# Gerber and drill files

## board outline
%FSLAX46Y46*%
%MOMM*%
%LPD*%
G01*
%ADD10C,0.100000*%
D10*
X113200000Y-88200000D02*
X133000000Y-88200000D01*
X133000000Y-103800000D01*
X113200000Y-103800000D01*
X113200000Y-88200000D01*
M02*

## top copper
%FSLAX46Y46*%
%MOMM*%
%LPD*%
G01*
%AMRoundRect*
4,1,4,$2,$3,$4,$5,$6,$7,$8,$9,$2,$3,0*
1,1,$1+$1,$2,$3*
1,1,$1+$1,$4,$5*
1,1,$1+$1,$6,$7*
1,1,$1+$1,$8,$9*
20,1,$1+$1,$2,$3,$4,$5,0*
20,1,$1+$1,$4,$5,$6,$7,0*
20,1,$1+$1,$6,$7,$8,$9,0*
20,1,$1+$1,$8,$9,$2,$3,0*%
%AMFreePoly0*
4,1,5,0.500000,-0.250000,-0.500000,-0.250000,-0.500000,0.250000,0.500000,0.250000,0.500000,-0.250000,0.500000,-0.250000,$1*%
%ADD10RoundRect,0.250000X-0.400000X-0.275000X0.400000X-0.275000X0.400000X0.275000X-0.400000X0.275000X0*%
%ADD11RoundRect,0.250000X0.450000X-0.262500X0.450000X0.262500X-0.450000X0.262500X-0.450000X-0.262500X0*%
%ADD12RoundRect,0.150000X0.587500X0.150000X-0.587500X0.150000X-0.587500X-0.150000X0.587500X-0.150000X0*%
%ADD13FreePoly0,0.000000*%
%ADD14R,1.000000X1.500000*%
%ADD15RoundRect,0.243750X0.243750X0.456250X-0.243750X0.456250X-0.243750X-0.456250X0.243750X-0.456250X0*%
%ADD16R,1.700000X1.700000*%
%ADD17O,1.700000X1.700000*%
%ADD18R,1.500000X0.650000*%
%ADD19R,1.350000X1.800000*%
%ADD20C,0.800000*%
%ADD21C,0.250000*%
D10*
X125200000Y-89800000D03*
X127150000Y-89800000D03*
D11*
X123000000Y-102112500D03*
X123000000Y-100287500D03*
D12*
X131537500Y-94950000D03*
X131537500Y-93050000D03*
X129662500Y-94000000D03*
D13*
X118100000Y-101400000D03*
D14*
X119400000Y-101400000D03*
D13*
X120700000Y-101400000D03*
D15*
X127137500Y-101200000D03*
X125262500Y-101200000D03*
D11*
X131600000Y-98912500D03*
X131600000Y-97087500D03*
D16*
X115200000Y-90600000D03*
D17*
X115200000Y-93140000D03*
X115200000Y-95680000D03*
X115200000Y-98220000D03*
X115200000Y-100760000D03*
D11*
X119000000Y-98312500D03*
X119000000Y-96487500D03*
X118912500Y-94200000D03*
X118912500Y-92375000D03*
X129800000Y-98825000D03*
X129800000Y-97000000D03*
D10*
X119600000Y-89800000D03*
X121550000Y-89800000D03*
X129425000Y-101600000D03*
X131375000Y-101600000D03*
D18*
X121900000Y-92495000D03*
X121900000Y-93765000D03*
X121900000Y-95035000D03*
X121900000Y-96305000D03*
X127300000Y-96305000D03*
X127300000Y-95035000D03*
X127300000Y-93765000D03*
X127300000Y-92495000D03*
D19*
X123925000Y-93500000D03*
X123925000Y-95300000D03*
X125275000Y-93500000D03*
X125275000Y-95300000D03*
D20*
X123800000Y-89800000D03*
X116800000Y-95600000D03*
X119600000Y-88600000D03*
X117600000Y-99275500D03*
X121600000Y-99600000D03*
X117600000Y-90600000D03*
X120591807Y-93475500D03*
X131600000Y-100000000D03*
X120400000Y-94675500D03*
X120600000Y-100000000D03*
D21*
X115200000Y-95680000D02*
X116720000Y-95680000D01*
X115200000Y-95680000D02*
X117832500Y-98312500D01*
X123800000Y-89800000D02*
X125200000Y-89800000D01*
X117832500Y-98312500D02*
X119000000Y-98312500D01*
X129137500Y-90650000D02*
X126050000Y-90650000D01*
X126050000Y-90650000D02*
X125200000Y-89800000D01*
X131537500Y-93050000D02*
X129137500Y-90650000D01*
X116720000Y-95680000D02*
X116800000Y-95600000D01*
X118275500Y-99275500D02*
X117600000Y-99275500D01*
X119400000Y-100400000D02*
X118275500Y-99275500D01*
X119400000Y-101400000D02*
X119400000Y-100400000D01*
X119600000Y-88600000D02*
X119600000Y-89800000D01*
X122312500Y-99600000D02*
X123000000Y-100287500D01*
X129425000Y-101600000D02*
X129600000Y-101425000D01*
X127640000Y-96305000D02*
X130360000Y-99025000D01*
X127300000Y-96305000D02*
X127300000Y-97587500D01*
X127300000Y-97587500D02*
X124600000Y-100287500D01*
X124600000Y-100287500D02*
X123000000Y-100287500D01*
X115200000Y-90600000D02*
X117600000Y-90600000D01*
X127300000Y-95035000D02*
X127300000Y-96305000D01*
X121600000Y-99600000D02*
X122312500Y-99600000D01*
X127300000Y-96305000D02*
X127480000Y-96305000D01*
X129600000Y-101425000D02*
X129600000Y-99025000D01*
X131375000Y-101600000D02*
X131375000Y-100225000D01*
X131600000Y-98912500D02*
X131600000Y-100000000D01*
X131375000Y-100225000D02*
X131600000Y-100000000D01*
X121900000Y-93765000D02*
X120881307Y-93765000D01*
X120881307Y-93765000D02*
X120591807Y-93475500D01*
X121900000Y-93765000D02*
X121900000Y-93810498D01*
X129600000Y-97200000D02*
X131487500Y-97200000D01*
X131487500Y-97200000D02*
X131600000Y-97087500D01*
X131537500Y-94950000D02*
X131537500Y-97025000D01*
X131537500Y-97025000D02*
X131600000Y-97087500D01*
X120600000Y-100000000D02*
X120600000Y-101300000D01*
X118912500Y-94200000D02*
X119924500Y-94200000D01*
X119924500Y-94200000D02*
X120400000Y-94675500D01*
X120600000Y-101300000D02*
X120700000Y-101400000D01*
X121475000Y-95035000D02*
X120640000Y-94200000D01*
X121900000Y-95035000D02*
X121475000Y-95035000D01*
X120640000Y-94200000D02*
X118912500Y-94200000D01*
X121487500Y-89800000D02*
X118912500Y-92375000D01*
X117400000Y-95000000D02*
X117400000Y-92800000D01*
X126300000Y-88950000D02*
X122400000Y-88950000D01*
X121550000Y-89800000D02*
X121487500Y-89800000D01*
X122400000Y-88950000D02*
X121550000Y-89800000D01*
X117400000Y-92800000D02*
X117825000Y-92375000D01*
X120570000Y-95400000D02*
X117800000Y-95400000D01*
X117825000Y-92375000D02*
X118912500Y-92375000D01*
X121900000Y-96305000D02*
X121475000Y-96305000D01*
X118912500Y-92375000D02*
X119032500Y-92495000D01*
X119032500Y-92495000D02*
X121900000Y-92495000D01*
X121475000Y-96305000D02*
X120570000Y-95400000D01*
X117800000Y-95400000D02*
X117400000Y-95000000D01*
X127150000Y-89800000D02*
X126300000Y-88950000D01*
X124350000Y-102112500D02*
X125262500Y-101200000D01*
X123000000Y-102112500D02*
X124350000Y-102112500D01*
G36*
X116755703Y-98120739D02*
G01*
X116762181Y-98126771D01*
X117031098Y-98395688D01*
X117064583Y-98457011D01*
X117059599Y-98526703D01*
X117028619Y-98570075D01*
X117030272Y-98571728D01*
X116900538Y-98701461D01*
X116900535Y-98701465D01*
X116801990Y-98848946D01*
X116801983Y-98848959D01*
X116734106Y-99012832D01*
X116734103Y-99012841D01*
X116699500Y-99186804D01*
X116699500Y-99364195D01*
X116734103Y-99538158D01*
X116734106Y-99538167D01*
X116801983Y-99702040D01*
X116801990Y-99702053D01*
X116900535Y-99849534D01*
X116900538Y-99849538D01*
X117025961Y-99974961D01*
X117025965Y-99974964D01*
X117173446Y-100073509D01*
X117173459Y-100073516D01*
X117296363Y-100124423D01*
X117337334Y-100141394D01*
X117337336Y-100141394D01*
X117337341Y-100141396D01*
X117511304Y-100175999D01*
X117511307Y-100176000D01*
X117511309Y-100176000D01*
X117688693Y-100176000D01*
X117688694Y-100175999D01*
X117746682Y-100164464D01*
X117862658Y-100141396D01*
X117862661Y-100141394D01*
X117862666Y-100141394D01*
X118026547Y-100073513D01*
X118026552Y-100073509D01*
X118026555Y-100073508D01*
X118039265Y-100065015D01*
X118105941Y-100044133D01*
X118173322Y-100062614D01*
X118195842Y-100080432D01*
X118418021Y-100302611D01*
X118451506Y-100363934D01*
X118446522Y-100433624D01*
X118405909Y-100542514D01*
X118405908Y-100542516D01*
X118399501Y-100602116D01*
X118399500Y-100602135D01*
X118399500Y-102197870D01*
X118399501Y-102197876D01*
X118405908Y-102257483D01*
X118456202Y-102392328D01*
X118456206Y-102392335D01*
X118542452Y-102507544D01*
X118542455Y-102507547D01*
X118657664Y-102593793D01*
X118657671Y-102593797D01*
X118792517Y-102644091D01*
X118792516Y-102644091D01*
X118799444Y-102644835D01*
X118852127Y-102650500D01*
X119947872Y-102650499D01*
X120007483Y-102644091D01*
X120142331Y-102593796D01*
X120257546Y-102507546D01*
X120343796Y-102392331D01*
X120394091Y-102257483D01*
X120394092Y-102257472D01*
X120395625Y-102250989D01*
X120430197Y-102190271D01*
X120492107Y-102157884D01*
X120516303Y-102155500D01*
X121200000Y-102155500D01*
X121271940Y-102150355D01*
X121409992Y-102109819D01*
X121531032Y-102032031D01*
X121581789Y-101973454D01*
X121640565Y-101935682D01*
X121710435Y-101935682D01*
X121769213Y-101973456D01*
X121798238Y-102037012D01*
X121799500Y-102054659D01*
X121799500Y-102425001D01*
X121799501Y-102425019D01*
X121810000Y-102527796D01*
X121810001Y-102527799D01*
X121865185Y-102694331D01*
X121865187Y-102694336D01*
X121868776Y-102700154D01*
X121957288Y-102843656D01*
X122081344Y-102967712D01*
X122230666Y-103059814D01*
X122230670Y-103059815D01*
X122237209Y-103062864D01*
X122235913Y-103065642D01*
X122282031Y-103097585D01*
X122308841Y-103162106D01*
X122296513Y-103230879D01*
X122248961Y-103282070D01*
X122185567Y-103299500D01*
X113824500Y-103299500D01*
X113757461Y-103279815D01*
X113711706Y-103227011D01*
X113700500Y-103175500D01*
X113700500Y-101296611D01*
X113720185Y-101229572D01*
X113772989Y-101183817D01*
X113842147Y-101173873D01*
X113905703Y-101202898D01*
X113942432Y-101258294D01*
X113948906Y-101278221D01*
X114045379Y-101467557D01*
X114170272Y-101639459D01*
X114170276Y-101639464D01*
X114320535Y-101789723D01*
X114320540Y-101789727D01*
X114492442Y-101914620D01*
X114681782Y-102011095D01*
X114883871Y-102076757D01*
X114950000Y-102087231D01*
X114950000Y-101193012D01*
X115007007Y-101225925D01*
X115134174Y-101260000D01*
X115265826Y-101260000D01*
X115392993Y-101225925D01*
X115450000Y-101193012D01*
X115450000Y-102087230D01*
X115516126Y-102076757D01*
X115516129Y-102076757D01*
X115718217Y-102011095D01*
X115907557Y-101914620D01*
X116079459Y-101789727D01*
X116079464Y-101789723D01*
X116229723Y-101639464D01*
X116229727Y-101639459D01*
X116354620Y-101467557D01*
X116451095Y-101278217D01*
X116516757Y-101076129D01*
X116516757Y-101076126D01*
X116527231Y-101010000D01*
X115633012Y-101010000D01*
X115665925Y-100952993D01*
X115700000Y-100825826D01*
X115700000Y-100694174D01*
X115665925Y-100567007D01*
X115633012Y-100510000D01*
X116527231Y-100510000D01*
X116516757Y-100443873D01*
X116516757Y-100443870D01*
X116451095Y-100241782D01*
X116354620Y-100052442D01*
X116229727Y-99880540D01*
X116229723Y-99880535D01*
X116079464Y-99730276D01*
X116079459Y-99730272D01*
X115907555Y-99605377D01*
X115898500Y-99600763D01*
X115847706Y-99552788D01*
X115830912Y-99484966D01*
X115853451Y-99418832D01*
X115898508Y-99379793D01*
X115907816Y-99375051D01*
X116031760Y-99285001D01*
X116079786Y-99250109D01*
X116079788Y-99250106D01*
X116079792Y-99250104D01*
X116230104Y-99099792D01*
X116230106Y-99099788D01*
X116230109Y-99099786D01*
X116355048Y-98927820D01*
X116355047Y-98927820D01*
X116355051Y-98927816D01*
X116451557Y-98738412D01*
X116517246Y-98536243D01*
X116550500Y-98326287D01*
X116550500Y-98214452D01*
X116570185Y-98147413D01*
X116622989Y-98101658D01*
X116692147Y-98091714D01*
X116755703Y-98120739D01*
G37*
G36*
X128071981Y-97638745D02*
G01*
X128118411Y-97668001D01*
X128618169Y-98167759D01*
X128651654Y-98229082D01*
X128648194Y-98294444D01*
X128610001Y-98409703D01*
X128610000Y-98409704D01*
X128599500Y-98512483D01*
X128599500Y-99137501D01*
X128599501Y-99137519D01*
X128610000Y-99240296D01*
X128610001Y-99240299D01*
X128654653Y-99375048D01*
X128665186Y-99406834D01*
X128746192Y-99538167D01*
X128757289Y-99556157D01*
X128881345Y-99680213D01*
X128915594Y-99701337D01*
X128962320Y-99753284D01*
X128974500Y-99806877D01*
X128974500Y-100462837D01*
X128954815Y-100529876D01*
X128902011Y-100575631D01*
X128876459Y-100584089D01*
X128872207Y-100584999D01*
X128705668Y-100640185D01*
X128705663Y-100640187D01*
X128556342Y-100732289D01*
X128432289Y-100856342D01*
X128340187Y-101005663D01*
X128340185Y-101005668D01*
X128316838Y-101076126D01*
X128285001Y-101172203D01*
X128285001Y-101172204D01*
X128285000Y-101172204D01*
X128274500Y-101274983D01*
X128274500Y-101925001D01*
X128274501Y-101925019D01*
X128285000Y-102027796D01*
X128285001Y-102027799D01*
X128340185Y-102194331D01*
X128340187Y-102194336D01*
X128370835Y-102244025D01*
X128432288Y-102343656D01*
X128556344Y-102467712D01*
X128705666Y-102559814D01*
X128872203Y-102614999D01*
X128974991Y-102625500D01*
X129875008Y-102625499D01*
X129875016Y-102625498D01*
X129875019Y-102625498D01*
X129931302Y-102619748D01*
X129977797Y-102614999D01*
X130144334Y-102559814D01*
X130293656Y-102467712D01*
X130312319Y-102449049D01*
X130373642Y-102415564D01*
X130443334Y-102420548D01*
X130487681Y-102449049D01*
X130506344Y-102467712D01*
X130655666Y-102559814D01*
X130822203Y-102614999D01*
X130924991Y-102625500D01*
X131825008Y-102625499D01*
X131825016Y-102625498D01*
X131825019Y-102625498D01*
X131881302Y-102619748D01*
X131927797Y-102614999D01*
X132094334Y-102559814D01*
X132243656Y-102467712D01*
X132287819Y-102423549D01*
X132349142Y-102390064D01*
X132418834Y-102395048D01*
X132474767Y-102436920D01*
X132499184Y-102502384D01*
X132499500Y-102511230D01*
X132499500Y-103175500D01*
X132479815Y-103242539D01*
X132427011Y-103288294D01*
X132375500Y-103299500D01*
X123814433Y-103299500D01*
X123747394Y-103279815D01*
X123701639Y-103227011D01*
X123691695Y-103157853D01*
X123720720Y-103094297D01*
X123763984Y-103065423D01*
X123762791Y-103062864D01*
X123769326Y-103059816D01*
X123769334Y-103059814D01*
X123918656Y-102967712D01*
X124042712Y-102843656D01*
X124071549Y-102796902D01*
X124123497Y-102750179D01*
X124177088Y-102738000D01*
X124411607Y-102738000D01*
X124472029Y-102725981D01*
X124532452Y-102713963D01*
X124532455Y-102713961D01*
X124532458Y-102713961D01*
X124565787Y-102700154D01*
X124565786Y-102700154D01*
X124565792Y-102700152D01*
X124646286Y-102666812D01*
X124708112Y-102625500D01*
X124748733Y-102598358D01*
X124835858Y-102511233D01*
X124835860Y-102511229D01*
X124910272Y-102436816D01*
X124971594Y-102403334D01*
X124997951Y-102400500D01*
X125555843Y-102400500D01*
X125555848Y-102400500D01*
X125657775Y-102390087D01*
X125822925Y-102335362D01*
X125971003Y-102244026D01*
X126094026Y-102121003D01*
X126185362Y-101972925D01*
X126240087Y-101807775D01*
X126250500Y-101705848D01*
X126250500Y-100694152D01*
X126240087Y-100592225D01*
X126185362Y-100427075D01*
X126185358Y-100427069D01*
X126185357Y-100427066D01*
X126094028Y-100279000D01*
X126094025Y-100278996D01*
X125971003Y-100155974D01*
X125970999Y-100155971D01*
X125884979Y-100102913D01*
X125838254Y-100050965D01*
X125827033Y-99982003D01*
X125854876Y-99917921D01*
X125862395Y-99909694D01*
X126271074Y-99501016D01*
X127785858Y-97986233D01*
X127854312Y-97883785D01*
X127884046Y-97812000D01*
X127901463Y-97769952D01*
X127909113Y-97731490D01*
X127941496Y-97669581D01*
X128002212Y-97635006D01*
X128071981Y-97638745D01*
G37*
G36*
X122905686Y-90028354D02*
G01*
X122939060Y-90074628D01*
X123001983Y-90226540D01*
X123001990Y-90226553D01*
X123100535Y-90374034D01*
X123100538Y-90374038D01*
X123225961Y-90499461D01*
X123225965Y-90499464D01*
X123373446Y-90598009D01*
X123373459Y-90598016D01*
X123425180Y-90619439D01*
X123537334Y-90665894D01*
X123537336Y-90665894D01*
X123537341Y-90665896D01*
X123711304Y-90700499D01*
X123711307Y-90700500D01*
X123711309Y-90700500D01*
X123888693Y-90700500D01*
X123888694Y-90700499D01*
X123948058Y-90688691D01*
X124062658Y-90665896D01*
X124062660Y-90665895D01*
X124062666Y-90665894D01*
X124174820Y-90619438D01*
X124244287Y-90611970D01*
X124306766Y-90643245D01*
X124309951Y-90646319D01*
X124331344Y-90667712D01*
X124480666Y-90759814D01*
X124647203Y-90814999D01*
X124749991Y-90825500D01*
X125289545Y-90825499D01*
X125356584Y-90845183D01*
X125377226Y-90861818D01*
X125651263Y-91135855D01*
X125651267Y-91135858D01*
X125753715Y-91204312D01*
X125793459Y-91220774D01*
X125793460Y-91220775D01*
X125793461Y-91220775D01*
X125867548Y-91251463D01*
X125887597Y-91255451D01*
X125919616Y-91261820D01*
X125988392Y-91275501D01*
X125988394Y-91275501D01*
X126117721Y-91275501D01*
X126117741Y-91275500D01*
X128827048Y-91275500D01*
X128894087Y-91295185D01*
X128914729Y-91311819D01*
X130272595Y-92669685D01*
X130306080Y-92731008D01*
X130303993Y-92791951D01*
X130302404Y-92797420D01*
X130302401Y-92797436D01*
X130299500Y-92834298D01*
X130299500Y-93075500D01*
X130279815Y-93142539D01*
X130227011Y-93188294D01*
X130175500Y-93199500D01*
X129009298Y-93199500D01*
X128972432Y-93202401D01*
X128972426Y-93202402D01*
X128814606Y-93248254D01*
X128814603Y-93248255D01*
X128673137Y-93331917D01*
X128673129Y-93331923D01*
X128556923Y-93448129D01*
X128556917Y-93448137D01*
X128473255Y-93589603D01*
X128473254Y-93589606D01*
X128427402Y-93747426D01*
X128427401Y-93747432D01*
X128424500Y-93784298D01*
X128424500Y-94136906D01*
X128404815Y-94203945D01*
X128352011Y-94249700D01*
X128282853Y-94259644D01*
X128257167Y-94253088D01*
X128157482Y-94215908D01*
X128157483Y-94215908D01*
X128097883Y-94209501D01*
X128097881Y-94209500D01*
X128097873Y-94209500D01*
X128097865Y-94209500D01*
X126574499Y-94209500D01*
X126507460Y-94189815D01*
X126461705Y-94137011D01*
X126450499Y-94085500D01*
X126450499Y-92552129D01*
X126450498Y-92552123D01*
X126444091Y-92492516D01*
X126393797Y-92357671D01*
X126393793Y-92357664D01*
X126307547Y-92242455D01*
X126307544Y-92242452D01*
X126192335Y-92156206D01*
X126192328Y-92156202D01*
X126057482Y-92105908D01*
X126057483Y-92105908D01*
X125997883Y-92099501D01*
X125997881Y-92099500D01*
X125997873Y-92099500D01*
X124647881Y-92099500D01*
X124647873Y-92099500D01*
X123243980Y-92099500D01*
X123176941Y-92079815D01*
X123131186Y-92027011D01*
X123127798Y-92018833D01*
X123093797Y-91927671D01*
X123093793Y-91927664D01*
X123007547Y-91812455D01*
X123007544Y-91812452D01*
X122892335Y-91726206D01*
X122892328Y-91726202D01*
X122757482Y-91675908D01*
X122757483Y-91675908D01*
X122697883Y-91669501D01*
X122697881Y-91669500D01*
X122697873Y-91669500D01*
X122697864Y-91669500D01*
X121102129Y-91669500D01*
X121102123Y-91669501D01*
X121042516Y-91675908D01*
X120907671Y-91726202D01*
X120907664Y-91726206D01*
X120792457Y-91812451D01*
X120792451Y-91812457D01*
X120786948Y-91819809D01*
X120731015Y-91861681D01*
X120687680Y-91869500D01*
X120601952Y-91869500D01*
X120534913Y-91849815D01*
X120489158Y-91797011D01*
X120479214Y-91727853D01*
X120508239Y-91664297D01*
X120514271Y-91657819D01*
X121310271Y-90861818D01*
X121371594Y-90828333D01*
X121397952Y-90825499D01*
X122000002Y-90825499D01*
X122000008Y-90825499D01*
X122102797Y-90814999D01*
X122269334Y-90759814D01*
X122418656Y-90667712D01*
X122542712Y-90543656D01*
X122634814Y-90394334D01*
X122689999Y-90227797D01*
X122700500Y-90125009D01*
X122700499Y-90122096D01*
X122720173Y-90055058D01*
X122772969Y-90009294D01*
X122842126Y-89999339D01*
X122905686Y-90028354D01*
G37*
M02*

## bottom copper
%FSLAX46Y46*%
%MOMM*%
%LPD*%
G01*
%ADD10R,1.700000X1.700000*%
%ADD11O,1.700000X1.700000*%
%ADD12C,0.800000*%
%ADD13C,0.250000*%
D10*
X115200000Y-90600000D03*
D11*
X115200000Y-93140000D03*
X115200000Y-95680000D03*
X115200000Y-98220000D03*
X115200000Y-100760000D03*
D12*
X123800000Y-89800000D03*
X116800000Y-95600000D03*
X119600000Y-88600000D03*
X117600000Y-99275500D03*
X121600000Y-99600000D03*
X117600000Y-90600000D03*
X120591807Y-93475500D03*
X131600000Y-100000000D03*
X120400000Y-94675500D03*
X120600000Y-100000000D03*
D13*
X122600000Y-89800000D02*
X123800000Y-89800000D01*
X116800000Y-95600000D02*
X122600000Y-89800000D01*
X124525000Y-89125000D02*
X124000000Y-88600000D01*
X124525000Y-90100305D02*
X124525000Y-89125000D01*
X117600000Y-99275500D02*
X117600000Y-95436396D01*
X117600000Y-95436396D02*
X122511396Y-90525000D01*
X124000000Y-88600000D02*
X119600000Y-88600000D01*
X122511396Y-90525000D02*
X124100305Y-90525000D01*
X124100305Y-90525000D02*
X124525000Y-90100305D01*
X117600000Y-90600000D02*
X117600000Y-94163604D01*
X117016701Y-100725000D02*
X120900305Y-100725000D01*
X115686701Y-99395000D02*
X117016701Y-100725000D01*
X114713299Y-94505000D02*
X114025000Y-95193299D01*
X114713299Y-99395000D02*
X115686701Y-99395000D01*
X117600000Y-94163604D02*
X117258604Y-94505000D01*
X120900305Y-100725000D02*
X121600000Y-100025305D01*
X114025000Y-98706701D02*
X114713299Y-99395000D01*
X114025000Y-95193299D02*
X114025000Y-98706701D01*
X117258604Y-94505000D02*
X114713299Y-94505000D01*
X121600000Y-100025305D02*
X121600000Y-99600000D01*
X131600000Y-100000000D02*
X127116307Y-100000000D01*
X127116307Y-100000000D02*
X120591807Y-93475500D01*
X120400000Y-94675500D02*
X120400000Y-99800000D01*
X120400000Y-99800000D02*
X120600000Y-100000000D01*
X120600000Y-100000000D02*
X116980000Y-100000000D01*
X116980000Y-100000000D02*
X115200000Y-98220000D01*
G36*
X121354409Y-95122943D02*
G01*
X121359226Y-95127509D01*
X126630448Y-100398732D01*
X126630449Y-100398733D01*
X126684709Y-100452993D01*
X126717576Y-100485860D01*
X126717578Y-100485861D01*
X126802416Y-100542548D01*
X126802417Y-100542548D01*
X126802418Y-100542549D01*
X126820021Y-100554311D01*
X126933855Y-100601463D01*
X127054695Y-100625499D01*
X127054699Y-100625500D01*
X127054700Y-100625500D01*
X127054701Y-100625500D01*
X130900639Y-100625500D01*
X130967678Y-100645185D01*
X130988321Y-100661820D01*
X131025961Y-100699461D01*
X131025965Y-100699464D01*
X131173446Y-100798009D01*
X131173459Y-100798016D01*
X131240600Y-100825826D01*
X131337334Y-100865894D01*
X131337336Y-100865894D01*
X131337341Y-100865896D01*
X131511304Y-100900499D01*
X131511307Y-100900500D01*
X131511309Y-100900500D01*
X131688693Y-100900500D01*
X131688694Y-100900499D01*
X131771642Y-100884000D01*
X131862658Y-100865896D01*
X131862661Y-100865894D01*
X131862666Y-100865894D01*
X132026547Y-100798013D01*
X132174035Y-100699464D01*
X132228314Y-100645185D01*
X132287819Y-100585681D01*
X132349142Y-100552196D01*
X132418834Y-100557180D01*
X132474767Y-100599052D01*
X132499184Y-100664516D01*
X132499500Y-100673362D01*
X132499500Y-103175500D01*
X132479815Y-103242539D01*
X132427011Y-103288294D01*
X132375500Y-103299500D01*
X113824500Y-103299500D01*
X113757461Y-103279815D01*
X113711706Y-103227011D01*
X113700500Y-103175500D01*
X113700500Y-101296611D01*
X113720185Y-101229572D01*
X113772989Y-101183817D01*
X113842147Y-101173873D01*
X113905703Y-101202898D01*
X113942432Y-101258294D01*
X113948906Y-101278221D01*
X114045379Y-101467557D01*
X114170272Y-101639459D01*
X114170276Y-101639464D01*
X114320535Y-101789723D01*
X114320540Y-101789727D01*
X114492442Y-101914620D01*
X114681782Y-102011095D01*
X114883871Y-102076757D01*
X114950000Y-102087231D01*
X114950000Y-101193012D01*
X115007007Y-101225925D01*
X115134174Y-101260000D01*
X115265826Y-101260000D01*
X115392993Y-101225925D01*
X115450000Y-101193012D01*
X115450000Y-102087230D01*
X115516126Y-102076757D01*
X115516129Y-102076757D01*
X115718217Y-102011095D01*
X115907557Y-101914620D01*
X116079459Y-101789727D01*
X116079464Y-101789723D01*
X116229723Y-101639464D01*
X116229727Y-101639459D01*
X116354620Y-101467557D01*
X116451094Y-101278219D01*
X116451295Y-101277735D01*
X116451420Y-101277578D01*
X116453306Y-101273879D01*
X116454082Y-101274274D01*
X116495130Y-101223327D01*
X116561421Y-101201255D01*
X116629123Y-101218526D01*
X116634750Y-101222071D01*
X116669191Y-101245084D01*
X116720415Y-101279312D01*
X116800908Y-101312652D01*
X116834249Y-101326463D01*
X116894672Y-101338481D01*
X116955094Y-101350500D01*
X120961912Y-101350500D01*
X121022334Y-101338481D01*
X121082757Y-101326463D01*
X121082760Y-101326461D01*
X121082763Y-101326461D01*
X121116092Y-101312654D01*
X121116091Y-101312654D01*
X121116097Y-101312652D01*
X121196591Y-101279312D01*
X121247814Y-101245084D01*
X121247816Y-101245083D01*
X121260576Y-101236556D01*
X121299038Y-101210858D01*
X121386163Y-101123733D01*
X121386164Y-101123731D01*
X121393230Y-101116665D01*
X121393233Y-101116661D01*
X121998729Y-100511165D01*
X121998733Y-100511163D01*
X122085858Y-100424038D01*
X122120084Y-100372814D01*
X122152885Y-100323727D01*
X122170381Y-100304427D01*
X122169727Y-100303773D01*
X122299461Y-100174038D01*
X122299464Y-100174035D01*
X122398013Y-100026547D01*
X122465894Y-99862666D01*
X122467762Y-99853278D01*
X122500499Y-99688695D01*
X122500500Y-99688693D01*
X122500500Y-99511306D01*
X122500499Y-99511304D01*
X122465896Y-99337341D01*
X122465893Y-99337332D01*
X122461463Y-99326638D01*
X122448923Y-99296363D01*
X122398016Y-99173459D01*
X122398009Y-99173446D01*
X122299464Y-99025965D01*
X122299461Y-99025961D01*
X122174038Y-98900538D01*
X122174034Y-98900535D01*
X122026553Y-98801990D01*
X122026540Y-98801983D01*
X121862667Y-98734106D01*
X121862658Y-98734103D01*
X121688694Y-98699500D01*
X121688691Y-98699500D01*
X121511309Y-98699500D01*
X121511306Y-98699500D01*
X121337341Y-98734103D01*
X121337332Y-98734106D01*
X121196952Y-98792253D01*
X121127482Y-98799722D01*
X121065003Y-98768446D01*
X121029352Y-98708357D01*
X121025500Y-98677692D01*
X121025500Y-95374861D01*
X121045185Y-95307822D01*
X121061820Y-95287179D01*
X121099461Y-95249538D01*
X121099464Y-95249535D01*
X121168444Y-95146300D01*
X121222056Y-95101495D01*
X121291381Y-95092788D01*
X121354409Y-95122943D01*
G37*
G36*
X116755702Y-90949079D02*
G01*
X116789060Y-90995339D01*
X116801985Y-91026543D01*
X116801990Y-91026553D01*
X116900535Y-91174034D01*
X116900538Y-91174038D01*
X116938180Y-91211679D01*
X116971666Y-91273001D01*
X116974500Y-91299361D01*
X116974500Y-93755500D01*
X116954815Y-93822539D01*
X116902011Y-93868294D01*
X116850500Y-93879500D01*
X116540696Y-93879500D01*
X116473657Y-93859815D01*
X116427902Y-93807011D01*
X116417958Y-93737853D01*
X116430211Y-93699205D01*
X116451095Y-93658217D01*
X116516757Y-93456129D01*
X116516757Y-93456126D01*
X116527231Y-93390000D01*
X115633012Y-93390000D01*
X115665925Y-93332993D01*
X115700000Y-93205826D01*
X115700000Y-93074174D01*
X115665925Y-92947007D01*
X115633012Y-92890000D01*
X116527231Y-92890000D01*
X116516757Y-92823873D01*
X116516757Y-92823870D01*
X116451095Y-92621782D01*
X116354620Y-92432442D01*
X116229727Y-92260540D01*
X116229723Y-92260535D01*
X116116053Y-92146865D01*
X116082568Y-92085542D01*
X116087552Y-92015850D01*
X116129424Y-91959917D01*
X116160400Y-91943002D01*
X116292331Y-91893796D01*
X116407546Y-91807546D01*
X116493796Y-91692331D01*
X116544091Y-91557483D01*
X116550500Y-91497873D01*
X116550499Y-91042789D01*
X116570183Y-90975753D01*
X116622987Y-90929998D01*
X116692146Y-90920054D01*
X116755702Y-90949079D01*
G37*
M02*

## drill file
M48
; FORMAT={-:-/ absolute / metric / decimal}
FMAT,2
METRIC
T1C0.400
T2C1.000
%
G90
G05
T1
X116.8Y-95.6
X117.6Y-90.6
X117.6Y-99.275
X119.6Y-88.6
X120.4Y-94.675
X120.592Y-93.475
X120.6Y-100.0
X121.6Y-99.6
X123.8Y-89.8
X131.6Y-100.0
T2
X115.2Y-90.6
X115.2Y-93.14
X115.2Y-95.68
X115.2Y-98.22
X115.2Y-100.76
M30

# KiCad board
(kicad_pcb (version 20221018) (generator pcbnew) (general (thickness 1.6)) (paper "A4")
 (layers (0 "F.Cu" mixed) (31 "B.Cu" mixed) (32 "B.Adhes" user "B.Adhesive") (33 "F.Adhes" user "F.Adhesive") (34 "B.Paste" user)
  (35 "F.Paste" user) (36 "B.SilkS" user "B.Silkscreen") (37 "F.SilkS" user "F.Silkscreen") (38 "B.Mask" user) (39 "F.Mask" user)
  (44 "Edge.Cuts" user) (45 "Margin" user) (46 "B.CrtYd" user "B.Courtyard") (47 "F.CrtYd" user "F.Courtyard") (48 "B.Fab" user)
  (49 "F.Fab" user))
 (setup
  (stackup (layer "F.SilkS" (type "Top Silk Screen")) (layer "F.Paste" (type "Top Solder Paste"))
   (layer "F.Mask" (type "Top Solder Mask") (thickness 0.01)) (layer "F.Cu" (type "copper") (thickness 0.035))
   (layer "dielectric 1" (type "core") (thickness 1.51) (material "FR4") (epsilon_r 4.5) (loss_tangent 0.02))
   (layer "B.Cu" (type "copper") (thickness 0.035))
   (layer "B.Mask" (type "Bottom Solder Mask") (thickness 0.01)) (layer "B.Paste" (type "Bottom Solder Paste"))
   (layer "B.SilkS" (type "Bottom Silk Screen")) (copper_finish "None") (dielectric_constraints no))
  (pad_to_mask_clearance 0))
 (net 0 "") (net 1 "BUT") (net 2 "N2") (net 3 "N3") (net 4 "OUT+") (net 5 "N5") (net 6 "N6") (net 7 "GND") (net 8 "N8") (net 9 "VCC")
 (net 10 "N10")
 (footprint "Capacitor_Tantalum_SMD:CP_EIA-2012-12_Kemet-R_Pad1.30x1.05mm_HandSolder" (layer "F.Cu") (at 126.175 89.8)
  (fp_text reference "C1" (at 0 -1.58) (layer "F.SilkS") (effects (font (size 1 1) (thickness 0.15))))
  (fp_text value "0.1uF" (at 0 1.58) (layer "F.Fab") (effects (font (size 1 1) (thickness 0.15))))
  (pad "1" smd roundrect (at -0.975 0) (size 1.3 1.05) (layers "F.Cu" "F.Paste" "F.Mask") (roundrect_rratio 0.2380952381) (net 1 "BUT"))
  (pad "2" smd roundrect (at 0.975 0) (size 1.3 1.05) (layers "F.Cu" "F.Paste" "F.Mask") (roundrect_rratio 0.2380952381) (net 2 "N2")))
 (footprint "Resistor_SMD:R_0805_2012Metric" (layer "F.Cu") (at 123 101.2 90)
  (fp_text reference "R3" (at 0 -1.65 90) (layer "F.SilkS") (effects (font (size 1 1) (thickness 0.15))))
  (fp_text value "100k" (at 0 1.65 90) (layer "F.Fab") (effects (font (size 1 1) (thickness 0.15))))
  (pad "1" smd roundrect (at -0.9125 0 90) (size 1.025 1.4) (layers "F.Cu" "F.Paste" "F.Mask") (roundrect_rratio 0.243902439) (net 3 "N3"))
  (pad "2" smd roundrect (at 0.9125 0 90) (size 1.025 1.4) (layers "F.Cu" "F.Paste" "F.Mask") (roundrect_rratio 0.243902439) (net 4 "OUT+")))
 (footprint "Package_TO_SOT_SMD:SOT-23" (layer "F.Cu") (at 130.6 94 180)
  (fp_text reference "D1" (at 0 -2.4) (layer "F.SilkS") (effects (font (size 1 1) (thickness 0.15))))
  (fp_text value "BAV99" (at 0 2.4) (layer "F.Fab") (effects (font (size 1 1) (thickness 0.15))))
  (pad "1" smd roundrect (at -0.9375 -0.95 180) (size 1.475 0.6) (layers "F.Cu" "F.Paste" "F.Mask") (roundrect_rratio 0.25) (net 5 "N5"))
  (pad "2" smd roundrect (at -0.9375 0.95 180) (size 1.475 0.6) (layers "F.Cu" "F.Paste" "F.Mask") (roundrect_rratio 0.25) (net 1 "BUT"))
  (pad "3" smd roundrect (at 0.9375 0 180) (size 1.475 0.6) (layers "F.Cu" "F.Paste" "F.Mask") (roundrect_rratio 0.25) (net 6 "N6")))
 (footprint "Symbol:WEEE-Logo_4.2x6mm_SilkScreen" (layer "F.Cu") (at 126 98.4)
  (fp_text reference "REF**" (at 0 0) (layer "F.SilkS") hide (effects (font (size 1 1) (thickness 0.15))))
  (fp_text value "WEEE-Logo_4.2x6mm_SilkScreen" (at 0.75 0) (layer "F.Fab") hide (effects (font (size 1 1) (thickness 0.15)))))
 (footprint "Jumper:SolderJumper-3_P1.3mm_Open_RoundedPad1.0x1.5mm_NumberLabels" (layer "F.Cu") (at 119.4 101.4)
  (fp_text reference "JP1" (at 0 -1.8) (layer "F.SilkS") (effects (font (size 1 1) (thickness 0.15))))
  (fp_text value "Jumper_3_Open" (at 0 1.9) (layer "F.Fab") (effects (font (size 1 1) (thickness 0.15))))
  (pad "1" smd custom (at -1.3 0) (size 1 0.5) (layers "F.Cu" "F.Mask") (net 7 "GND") (zone_connect 2) (thermal_bridge_angle 45)
   (options (clearance outline) (anchor rect)) (primitives))
  (pad "2" smd rect (at 0 0) (size 1 1.5) (layers "F.Cu" "F.Mask") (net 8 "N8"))
  (pad "3" smd custom (at 1.3 0) (size 1 0.5) (layers "F.Cu" "F.Mask") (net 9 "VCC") (zone_connect 2) (thermal_bridge_angle 45)
   (options (clearance outline) (anchor rect)) (primitives)))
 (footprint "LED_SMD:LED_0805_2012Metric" (layer "F.Cu") (at 126.2 101.2 180)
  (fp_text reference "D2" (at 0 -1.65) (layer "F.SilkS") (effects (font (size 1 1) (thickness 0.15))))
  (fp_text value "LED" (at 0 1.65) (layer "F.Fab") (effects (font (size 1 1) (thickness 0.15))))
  (pad "1" smd roundrect (at -0.9375 0 180) (size 0.975 1.4) (layers "F.Cu" "F.Paste" "F.Mask") (roundrect_rratio 0.25) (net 7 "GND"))
  (pad "2" smd roundrect (at 0.9375 0 180) (size 0.975 1.4) (layers "F.Cu" "F.Paste" "F.Mask") (roundrect_rratio 0.25) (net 3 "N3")))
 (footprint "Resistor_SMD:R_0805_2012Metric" (layer "F.Cu") (at 131.6 98 90)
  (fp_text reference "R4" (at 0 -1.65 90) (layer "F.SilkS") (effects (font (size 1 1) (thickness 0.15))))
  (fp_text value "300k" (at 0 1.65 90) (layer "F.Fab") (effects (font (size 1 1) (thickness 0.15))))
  (pad "1" smd roundrect (at -0.9125 0 90) (size 1.025 1.4) (layers "F.Cu" "F.Paste" "F.Mask") (roundrect_rratio 0.243902439) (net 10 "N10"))
  (pad "2" smd roundrect (at 0.9125 0 90) (size 1.025 1.4) (layers "F.Cu" "F.Paste" "F.Mask") (roundrect_rratio 0.243902439) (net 5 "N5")))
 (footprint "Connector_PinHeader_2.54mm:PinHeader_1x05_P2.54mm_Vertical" (layer "F.Cu") (at 115.2 90.6)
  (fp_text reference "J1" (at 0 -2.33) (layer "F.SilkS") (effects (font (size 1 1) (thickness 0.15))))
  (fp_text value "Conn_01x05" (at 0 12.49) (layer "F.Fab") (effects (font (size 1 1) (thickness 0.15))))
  (pad "1" thru_hole rect (at 0 0) (size 1.7 1.7) (drill 1) (layers "*.Cu" "*.Mask") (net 4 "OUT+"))
  (pad "2" thru_hole oval (at 0 2.54) (size 1.7 1.7) (drill 1) (layers "*.Cu" "*.Mask") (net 7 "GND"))
  (pad "3" thru_hole oval (at 0 5.08) (size 1.7 1.7) (drill 1) (layers "*.Cu" "*.Mask") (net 1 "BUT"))
  (pad "4" thru_hole oval (at 0 7.62) (size 1.7 1.7) (drill 1) (layers "*.Cu" "*.Mask") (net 9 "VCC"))
  (pad "5" thru_hole oval (at 0 10.16) (size 1.7 1.7) (drill 1) (layers "*.Cu" "*.Mask") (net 7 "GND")))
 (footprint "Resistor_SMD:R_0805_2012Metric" (layer "F.Cu") (at 119 97.4 90)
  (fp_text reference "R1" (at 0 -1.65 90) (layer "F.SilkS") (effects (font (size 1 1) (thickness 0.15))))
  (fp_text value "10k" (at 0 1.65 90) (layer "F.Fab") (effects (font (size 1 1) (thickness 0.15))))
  (pad "1" smd roundrect (at -0.9125 0 90) (size 1.025 1.4) (layers "F.Cu" "F.Paste" "F.Mask") (roundrect_rratio 0.243902439) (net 1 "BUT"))
  (pad "2" smd roundrect (at 0.9125 0 90) (size 1.025 1.4) (layers "F.Cu" "F.Paste" "F.Mask") (roundrect_rratio 0.243902439) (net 9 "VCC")))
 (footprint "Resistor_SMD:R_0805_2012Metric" (layer "F.Cu") (at 118.9125 93.2875 90)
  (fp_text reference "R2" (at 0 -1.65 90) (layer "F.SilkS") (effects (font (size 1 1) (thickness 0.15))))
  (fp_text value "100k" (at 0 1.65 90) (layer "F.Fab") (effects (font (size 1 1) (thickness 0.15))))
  (pad "1" smd roundrect (at -0.9125 0 90) (size 1.025 1.4) (layers "F.Cu" "F.Paste" "F.Mask") (roundrect_rratio 0.243902439) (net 9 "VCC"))
  (pad "2" smd roundrect (at 0.9125 0 90) (size 1.025 1.4) (layers "F.Cu" "F.Paste" "F.Mask") (roundrect_rratio 0.243902439) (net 2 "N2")))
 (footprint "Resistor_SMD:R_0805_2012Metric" (layer "F.Cu") (at 129.8 97.9125 90)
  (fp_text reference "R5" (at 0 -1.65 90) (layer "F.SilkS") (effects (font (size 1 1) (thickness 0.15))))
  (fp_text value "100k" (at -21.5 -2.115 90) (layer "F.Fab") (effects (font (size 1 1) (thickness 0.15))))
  (pad "1" smd roundrect (at -0.9125 0 90) (size 1.025 1.4) (layers "F.Cu" "F.Paste" "F.Mask") (roundrect_rratio 0.243902439) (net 4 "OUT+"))
  (pad "2" smd roundrect (at 0.9125 0 90) (size 1.025 1.4) (layers "F.Cu" "F.Paste" "F.Mask") (roundrect_rratio 0.243902439) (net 5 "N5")))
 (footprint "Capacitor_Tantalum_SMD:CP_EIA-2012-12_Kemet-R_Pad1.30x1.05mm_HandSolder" (layer "F.Cu") (at 120.575 89.8)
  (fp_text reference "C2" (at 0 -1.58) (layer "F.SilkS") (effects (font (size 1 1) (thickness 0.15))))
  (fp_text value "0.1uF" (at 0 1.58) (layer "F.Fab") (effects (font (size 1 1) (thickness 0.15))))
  (pad "1" smd roundrect (at -0.975 0) (size 1.3 1.05) (layers "F.Cu" "F.Paste" "F.Mask") (roundrect_rratio 0.2380952381) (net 8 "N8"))
  (pad "2" smd roundrect (at 0.975 0) (size 1.3 1.05) (layers "F.Cu" "F.Paste" "F.Mask") (roundrect_rratio 0.2380952381) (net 2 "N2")))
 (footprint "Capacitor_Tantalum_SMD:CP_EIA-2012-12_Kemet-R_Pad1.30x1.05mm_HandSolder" (layer "F.Cu") (at 130.4 101.6)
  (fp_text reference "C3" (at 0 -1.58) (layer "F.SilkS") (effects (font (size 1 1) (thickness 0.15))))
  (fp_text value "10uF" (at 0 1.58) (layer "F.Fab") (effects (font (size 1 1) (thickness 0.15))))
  (pad "1" smd roundrect (at -0.975 0) (size 1.3 1.05) (layers "F.Cu" "F.Paste" "F.Mask") (roundrect_rratio 0.2380952381) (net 4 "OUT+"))
  (pad "2" smd roundrect (at 0.975 0) (size 1.3 1.05) (layers "F.Cu" "F.Paste" "F.Mask") (roundrect_rratio 0.2380952381) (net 10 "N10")))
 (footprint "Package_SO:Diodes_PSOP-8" (layer "F.Cu") (at 124.6 94.4)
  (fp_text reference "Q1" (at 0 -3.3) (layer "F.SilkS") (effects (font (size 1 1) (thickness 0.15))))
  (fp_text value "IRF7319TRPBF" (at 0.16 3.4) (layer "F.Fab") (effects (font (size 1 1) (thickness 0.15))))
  (pad "1" smd rect (at -2.7 -1.905) (size 1.5 0.65) (layers "F.Cu" "F.Paste" "F.Mask") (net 2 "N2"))
  (pad "2" smd rect (at -2.7 -0.635) (size 1.5 0.65) (layers "F.Cu" "F.Paste" "F.Mask") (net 10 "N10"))
  (pad "3" smd rect (at -2.7 0.635) (size 1.5 0.65) (layers "F.Cu" "F.Paste" "F.Mask") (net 9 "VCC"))
  (pad "4" smd rect (at -2.7 1.905) (size 1.5 0.65) (layers "F.Cu" "F.Paste" "F.Mask") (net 2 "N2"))
  (pad "5" smd rect (at 2.7 1.905) (size 1.5 0.65) (layers "F.Cu" "F.Paste" "F.Mask") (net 4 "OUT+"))
  (pad "6" smd rect (at 2.7 0.635) (size 1.5 0.65) (layers "F.Cu" "F.Paste" "F.Mask") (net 4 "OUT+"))
  (pad "7" smd rect (at 2.7 -0.635) (size 1.5 0.65) (layers "F.Cu" "F.Paste" "F.Mask") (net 7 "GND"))
  (pad "8" smd rect (at 2.7 -1.905) (size 1.5 0.65) (layers "F.Cu" "F.Paste" "F.Mask") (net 7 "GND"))
  (pad "9" smd rect (at -0.675 -0.9) (size 1.35 1.8) (layers "F.Cu" "F.Paste" "F.Mask") (solder_paste_margin_ratio -0.2))
  (pad "9" smd rect (at -0.675 0.9) (size 1.35 1.8) (layers "F.Cu" "F.Paste" "F.Mask") (solder_paste_margin_ratio -0.2))
  (pad "9" smd rect (at 0.675 -0.9) (size 1.35 1.8) (layers "F.Cu" "F.Paste" "F.Mask") (solder_paste_margin_ratio -0.2))
  (pad "9" smd rect (at 0.675 0.9) (size 1.35 1.8) (layers "F.Cu" "F.Paste" "F.Mask") (solder_paste_margin_ratio -0.2)))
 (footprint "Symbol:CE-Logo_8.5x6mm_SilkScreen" (layer "B.Cu") (at 127.6 92 180)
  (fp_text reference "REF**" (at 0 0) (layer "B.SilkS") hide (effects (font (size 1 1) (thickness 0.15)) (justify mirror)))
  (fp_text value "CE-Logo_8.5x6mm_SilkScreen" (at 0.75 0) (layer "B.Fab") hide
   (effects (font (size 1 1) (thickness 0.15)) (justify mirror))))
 (gr_rect (start 113.2 88.2) (end 133 103.8) (stroke (width 0.1) (type default)) (fill none) (layer "Edge.Cuts"))
 (segment (start 115.2 95.68) (end 116.72 95.68) (width 0.25) (layer "F.Cu") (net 1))
 (segment (start 115.2 95.68) (end 117.8325 98.3125) (width 0.25) (layer "F.Cu") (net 1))
 (segment (start 123.8 89.8) (end 125.2 89.8) (width 0.25) (layer "F.Cu") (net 1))
 (segment (start 117.8325 98.3125) (end 119 98.3125) (width 0.25) (layer "F.Cu") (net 1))
 (segment (start 129.1375 90.65) (end 126.05 90.65) (width 0.25) (layer "F.Cu") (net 1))
 (segment (start 126.05 90.65) (end 125.2 89.8) (width 0.25) (layer "F.Cu") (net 1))
 (segment (start 131.5375 93.05) (end 129.1375 90.65) (width 0.25) (layer "F.Cu") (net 1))
 (segment (start 116.72 95.68) (end 116.8 95.6) (width 0.25) (layer "F.Cu") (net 1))
 (via (at 123.8 89.8) (size 0.8) (drill 0.4) (layers "F.Cu" "B.Cu") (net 1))
 (via (at 116.8 95.6) (size 0.8) (drill 0.4) (layers "F.Cu" "B.Cu") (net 1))
 (segment (start 122.6 89.8) (end 123.8 89.8) (width 0.25) (layer "B.Cu") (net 1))
 (segment (start 116.8 95.6) (end 122.6 89.8) (width 0.25) (layer "B.Cu") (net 1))
 (segment (start 118.2755 99.2755) (end 117.6 99.2755) (width 0.25) (layer "F.Cu") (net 8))
 (segment (start 119.4 100.4) (end 118.2755 99.2755) (width 0.25) (layer "F.Cu") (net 8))
 (segment (start 119.4 101.4) (end 119.4 100.4) (width 0.25) (layer "F.Cu") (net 8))
 (segment (start 119.6 88.6) (end 119.6 89.8) (width 0.25) (layer "F.Cu") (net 8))
 (via (at 119.6 88.6) (size 0.8) (drill 0.4) (layers "F.Cu" "B.Cu") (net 8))
 (via (at 117.6 99.2755) (size 0.8) (drill 0.4) (layers "F.Cu" "B.Cu") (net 8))
 (segment (start 124.525 89.125) (end 124 88.6) (width 0.25) (layer "B.Cu") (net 8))
 (segment (start 124.525 90.100305) (end 124.525 89.125) (width 0.25) (layer "B.Cu") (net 8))
 (segment (start 117.6 99.2755) (end 117.6 95.436396) (width 0.25) (layer "B.Cu") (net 8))
 (segment (start 117.6 95.436396) (end 122.511396 90.525) (width 0.25) (layer "B.Cu") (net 8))
 (segment (start 124 88.6) (end 119.6 88.6) (width 0.25) (layer "B.Cu") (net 8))
 (segment (start 122.511396 90.525) (end 124.100305 90.525) (width 0.25) (layer "B.Cu") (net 8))
 (segment (start 124.100305 90.525) (end 124.525 90.100305) (width 0.25) (layer "B.Cu") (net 8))
 (segment (start 122.3125 99.6) (end 123 100.2875) (width 0.25) (layer "F.Cu") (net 4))
 (segment (start 129.425 101.6) (end 129.6 101.425) (width 0.25) (layer "F.Cu") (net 4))
 (segment (start 127.64 96.305) (end 130.36 99.025) (width 0.25) (layer "F.Cu") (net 4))
 (segment (start 127.3 96.305) (end 127.3 97.5875) (width 0.25) (layer "F.Cu") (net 4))
 (segment (start 127.3 97.5875) (end 124.6 100.2875) (width 0.25) (layer "F.Cu") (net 4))
 (segment (start 124.6 100.2875) (end 123 100.2875) (width 0.25) (layer "F.Cu") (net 4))
 (segment (start 115.2 90.6) (end 117.6 90.6) (width 0.25) (layer "F.Cu") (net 4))
 (segment (start 127.3 95.035) (end 127.3 96.305) (width 0.25) (layer "F.Cu") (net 4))
 (segment (start 121.6 99.6) (end 122.3125 99.6) (width 0.25) (layer "F.Cu") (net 4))
 (segment (start 127.3 96.305) (end 127.48 96.305) (width 0.25) (layer "F.Cu") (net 4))
 (segment (start 129.6 101.425) (end 129.6 99.025) (width 0.25) (layer "F.Cu") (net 4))
 (via (at 121.6 99.6) (size 0.8) (drill 0.4) (layers "F.Cu" "B.Cu") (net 4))
 (via (at 117.6 90.6) (size 0.8) (drill 0.4) (layers "F.Cu" "B.Cu") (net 4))
 (segment (start 117.6 90.6) (end 117.6 94.163604) (width 0.25) (layer "B.Cu") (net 4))
 (segment (start 117.016701 100.725) (end 120.900305 100.725) (width 0.25) (layer "B.Cu") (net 4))
 (segment (start 115.686701 99.395) (end 117.016701 100.725) (width 0.25) (layer "B.Cu") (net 4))
 (segment (start 114.713299 94.505) (end 114.025 95.193299) (width 0.25) (layer "B.Cu") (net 4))
 (segment (start 114.713299 99.395) (end 115.686701 99.395) (width 0.25) (layer "B.Cu") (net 4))
 (segment (start 117.6 94.163604) (end 117.258604 94.505) (width 0.25) (layer "B.Cu") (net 4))
 (segment (start 120.900305 100.725) (end 121.6 100.025305) (width 0.25) (layer "B.Cu") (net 4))
 (segment (start 114.025 98.706701) (end 114.713299 99.395) (width 0.25) (layer "B.Cu") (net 4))
 (segment (start 114.025 95.193299) (end 114.025 98.706701) (width 0.25) (layer "B.Cu") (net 4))
 (segment (start 117.258604 94.505) (end 114.713299 94.505) (width 0.25) (layer "B.Cu") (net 4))
 (segment (start 121.6 100.025305) (end 121.6 99.6) (width 0.25) (layer "B.Cu") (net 4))
 (segment (start 131.375 101.6) (end 131.375 100.225) (width 0.25) (layer "F.Cu") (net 10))
 (segment (start 131.6 98.9125) (end 131.6 100) (width 0.25) (layer "F.Cu") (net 10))
 (segment (start 131.375 100.225) (end 131.6 100) (width 0.25) (layer "F.Cu") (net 10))
 (segment (start 121.9 93.765) (end 120.881307 93.765) (width 0.25) (layer "F.Cu") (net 10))
 (segment (start 120.881307 93.765) (end 120.591807 93.4755) (width 0.25) (layer "F.Cu") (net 10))
 (segment (start 121.9 93.765) (end 121.9 93.810498) (width 0.25) (layer "F.Cu") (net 10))
 (via (at 120.591807 93.4755) (size 0.8) (drill 0.4) (layers "F.Cu" "B.Cu") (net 10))
 (via (at 131.6 100) (size 0.8) (drill 0.4) (layers "F.Cu" "B.Cu") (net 10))
 (segment (start 131.6 100) (end 127.116307 100) (width 0.25) (layer "B.Cu") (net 10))
 (segment (start 127.116307 100) (end 120.591807 93.4755) (width 0.25) (layer "B.Cu") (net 10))
 (segment (start 129.6 97.2) (end 131.4875 97.2) (width 0.25) (layer "F.Cu") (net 5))
 (segment (start 131.4875 97.2) (end 131.6 97.0875) (width 0.25) (layer "F.Cu") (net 5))
 (segment (start 131.5375 94.95) (end 131.5375 97.025) (width 0.25) (layer "F.Cu") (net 5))
 (segment (start 131.5375 97.025) (end 131.6 97.0875) (width 0.25) (layer "F.Cu") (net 5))
 (segment (start 120.6 100) (end 120.6 101.3) (width 0.25) (layer "F.Cu") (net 9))
 (segment (start 118.9125 94.2) (end 119.9245 94.2) (width 0.25) (layer "F.Cu") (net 9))
 (segment (start 119.9245 94.2) (end 120.4 94.6755) (width 0.25) (layer "F.Cu") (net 9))
 (segment (start 120.6 101.3) (end 120.7 101.4) (width 0.25) (layer "F.Cu") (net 9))
 (segment (start 121.475 95.035) (end 120.64 94.2) (width 0.25) (layer "F.Cu") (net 9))
 (segment (start 121.9 95.035) (end 121.475 95.035) (width 0.25) (layer "F.Cu") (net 9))
 (segment (start 120.64 94.2) (end 118.9125 94.2) (width 0.25) (layer "F.Cu") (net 9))
 (via (at 120.4 94.6755) (size 0.8) (drill 0.4) (layers "F.Cu" "B.Cu") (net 9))
 (via (at 120.6 100) (size 0.8) (drill 0.4) (layers "F.Cu" "B.Cu") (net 9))
 (segment (start 120.4 94.6755) (end 120.4 99.8) (width 0.25) (layer "B.Cu") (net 9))
 (segment (start 120.4 99.8) (end 120.6 100) (width 0.25) (layer "B.Cu") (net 9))
 (segment (start 120.6 100) (end 116.98 100) (width 0.25) (layer "B.Cu") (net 9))
 (segment (start 116.98 100) (end 115.2 98.22) (width 0.25) (layer "B.Cu") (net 9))
 (segment (start 121.4875 89.8) (end 118.9125 92.375) (width 0.25) (layer "F.Cu") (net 2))
 (segment (start 117.4 95) (end 117.4 92.8) (width 0.25) (layer "F.Cu") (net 2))
 (segment (start 126.3 88.95) (end 122.4 88.95) (width 0.25) (layer "F.Cu") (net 2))
 (segment (start 121.55 89.8) (end 121.4875 89.8) (width 0.25) (layer "F.Cu") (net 2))
 (segment (start 122.4 88.95) (end 121.55 89.8) (width 0.25) (layer "F.Cu") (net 2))
 (segment (start 117.4 92.8) (end 117.825 92.375) (width 0.25) (layer "F.Cu") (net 2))
 (segment (start 120.57 95.4) (end 117.8 95.4) (width 0.25) (layer "F.Cu") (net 2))
 (segment (start 117.825 92.375) (end 118.9125 92.375) (width 0.25) (layer "F.Cu") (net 2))
 (segment (start 121.9 96.305) (end 121.475 96.305) (width 0.25) (layer "F.Cu") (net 2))
 (segment (start 118.9125 92.375) (end 119.0325 92.495) (width 0.25) (layer "F.Cu") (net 2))
 (segment (start 119.0325 92.495) (end 121.9 92.495) (width 0.25) (layer "F.Cu") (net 2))
 (segment (start 121.475 96.305) (end 120.57 95.4) (width 0.25) (layer "F.Cu") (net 2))
 (segment (start 117.8 95.4) (end 117.4 95) (width 0.25) (layer "F.Cu") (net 2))
 (segment (start 127.15 89.8) (end 126.3 88.95) (width 0.25) (layer "F.Cu") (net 2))
 (segment (start 124.35 102.1125) (end 125.2625 101.2) (width 0.25) (layer "F.Cu") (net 3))
 (segment (start 123 102.1125) (end 124.35 102.1125) (width 0.25) (layer "F.Cu") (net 3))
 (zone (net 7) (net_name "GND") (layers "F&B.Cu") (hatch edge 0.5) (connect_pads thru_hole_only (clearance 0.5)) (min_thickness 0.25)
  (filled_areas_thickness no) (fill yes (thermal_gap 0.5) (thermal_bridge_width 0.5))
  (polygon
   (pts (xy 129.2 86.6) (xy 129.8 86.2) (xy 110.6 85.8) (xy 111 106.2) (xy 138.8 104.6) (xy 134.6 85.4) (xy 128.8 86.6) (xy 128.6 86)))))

